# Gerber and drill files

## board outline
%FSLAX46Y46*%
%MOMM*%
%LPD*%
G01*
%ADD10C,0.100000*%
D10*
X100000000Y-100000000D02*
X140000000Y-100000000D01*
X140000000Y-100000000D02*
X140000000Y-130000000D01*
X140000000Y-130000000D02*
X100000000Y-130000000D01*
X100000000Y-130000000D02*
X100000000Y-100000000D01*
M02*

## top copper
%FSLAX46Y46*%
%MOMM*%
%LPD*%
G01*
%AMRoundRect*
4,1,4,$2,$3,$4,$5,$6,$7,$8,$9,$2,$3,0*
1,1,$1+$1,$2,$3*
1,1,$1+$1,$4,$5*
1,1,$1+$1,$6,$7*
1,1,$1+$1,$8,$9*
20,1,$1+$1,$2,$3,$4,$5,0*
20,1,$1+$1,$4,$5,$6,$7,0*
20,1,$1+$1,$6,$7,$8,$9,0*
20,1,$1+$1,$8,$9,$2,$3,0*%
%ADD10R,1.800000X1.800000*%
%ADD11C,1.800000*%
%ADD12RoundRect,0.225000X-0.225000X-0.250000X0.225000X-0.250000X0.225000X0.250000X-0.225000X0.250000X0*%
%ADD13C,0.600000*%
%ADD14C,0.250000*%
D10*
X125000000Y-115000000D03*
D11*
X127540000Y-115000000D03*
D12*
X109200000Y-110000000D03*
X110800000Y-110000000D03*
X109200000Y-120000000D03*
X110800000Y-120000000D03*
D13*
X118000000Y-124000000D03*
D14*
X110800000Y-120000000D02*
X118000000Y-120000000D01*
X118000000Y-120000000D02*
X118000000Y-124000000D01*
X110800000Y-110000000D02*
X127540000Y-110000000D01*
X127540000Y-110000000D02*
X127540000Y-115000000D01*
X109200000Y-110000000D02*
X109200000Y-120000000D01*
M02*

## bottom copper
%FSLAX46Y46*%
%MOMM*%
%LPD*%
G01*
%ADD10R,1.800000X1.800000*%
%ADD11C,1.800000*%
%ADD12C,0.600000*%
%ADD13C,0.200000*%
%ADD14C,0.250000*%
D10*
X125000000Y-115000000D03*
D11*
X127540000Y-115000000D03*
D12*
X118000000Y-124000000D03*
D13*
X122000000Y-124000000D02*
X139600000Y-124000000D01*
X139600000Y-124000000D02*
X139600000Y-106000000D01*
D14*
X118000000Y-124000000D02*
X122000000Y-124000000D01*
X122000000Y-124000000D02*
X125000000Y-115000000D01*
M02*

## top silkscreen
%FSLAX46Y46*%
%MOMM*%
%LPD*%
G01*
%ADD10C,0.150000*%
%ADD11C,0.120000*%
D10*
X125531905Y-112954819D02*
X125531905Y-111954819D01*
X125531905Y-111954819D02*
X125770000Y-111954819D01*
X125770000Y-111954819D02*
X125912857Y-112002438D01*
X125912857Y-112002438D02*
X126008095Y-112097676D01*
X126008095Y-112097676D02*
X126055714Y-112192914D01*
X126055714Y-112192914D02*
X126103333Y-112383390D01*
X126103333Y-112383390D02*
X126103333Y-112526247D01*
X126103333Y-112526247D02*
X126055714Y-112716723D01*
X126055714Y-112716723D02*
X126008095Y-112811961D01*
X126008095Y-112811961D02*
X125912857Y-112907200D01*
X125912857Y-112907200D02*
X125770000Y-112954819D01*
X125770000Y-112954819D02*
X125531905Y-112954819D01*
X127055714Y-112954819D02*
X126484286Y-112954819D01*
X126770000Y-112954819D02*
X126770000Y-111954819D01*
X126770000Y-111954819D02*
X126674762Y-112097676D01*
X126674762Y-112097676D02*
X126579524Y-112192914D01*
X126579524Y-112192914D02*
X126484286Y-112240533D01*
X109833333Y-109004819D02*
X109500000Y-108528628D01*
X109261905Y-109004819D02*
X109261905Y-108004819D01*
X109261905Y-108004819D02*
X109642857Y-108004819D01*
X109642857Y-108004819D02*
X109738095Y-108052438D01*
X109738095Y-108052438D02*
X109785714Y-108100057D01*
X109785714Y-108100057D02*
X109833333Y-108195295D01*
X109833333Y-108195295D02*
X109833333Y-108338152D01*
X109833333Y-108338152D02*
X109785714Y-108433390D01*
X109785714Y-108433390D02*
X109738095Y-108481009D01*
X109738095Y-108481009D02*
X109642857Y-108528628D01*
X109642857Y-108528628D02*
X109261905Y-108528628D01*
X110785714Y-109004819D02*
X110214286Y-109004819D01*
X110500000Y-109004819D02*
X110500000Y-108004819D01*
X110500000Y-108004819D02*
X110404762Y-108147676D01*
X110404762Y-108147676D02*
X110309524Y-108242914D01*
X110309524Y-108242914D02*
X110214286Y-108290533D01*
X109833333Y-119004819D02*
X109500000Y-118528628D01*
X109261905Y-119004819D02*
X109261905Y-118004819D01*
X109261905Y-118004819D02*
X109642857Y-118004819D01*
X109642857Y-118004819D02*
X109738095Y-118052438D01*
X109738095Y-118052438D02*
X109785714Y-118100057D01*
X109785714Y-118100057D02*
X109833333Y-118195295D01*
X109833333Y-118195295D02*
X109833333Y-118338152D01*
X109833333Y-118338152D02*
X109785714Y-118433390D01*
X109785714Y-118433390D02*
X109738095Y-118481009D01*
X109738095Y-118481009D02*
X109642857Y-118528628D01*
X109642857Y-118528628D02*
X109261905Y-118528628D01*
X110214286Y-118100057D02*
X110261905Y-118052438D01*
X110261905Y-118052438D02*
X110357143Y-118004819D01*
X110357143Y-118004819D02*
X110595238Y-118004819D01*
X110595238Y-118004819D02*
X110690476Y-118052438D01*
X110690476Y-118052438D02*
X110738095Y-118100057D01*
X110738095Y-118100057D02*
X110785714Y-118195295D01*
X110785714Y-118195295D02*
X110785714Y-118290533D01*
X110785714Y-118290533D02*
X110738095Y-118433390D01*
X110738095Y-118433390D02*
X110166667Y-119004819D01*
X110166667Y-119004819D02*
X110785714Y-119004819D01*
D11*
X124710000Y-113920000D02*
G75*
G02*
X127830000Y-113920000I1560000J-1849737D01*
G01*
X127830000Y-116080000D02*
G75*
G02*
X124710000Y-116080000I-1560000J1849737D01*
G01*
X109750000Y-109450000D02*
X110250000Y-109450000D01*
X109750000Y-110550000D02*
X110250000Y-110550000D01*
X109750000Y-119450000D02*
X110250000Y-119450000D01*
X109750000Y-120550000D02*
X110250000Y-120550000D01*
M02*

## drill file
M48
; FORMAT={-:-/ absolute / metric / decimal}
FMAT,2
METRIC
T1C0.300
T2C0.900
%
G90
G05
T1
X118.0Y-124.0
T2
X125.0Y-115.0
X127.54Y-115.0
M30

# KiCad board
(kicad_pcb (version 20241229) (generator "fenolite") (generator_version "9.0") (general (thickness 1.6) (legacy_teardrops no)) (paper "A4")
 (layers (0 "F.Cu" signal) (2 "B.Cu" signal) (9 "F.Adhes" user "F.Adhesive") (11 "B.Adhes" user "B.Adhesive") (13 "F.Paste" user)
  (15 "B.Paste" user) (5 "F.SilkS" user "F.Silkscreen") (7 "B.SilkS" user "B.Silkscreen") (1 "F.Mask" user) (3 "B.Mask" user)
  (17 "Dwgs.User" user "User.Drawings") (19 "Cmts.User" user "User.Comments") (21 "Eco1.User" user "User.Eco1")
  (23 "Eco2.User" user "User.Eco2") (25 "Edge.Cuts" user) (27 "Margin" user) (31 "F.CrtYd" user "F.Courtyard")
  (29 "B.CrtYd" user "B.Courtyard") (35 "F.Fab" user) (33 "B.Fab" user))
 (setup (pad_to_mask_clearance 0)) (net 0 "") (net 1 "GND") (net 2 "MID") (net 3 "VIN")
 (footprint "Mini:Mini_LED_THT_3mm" (layer "F.Cu") (at 125 115)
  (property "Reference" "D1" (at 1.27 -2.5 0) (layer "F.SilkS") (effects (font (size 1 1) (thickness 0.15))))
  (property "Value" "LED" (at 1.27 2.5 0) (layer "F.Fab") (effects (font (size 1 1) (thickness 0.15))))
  (fp_arc (start -0.29 -1.08) (mid 1.27 -1.65) (end 2.83 -1.08) (stroke (width 0.12) (type solid)) (layer "F.SilkS"))
  (fp_arc (start 2.83 1.08) (mid 1.27 1.65) (end -0.29 1.08) (stroke (width 0.12) (type solid)) (layer "F.SilkS"))
  (pad "1" thru_hole rect (at 0 0) (size 1.8 1.8) (drill 0.9) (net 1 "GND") (layers "*.Cu" "*.Mask") (remove_unused_layers no))
  (pad "2" thru_hole circle (at 2.54 0) (size 1.8 1.8) (drill 0.9) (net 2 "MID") (layers "*.Cu" "*.Mask") (remove_unused_layers no)))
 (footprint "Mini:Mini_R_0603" (layer "F.Cu") (at 110 110)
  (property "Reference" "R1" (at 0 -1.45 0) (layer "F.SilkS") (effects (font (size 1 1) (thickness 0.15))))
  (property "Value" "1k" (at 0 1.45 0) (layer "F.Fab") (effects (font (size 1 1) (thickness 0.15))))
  (fp_line (start -0.25 -0.55) (end 0.25 -0.55) (stroke (width 0.12) (type solid)) (layer "F.SilkS"))
  (fp_line (start -0.25 0.55) (end 0.25 0.55) (stroke (width 0.12) (type solid)) (layer "F.SilkS"))
  (pad "1" smd roundrect (at -0.8 0) (size 0.9 0.95) (layers "F.Cu" "F.Mask" "F.Paste") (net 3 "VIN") (roundrect_rratio 0.25))
  (pad "2" smd roundrect (at 0.8 0) (size 0.9 0.95) (layers "F.Cu" "F.Mask" "F.Paste") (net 2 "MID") (roundrect_rratio 0.25)))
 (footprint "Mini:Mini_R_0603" (layer "F.Cu") (at 110 120)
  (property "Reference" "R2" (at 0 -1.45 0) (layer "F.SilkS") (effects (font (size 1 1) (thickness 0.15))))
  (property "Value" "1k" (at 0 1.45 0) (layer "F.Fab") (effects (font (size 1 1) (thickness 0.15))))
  (fp_line (start -0.25 -0.55) (end 0.25 -0.55) (stroke (width 0.12) (type solid)) (layer "F.SilkS"))
  (fp_line (start -0.25 0.55) (end 0.25 0.55) (stroke (width 0.12) (type solid)) (layer "F.SilkS"))
  (pad "1" smd roundrect (at -0.8 0) (size 0.9 0.95) (layers "F.Cu" "F.Mask" "F.Paste") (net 3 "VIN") (roundrect_rratio 0.25))
  (pad "2" smd roundrect (at 0.8 0) (size 0.9 0.95) (layers "F.Cu" "F.Mask" "F.Paste") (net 1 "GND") (roundrect_rratio 0.25)))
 (gr_line (start 100 100) (end 140 100) (stroke (width 0.1) (type solid)) (layer "Edge.Cuts"))
 (gr_line (start 140 100) (end 140 130) (stroke (width 0.1) (type solid)) (layer "Edge.Cuts"))
 (gr_line (start 140 130) (end 100 130) (stroke (width 0.1) (type solid)) (layer "Edge.Cuts"))
 (gr_line (start 100 130) (end 100 100) (stroke (width 0.1) (type solid)) (layer "Edge.Cuts"))
 (segment (start 122 124) (end 139.6 124) (width 0.2) (layer "B.Cu") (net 1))
 (segment (start 139.6 124) (end 139.6 106) (width 0.2) (layer "B.Cu") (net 1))
 (segment (start 110.8 120) (end 118 120) (width 0.25) (layer "F.Cu") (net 1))
 (segment (start 118 120) (end 118 124) (width 0.25) (layer "F.Cu") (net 1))
 (segment (start 118 124) (end 122 124) (width 0.25) (layer "B.Cu") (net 1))
 (segment (start 122 124) (end 125 115) (width 0.25) (layer "B.Cu") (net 1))
 (segment (start 110.8 110) (end 127.54 110) (width 0.25) (layer "F.Cu") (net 2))
 (segment (start 127.54 110) (end 127.54 115) (width 0.25) (layer "F.Cu") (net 2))
 (segment (start 109.2 110) (end 109.2 120) (width 0.25) (layer "F.Cu") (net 3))
 (via (at 118 124) (size 0.6) (drill 0.3) (layers "F.Cu" "B.Cu") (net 1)))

